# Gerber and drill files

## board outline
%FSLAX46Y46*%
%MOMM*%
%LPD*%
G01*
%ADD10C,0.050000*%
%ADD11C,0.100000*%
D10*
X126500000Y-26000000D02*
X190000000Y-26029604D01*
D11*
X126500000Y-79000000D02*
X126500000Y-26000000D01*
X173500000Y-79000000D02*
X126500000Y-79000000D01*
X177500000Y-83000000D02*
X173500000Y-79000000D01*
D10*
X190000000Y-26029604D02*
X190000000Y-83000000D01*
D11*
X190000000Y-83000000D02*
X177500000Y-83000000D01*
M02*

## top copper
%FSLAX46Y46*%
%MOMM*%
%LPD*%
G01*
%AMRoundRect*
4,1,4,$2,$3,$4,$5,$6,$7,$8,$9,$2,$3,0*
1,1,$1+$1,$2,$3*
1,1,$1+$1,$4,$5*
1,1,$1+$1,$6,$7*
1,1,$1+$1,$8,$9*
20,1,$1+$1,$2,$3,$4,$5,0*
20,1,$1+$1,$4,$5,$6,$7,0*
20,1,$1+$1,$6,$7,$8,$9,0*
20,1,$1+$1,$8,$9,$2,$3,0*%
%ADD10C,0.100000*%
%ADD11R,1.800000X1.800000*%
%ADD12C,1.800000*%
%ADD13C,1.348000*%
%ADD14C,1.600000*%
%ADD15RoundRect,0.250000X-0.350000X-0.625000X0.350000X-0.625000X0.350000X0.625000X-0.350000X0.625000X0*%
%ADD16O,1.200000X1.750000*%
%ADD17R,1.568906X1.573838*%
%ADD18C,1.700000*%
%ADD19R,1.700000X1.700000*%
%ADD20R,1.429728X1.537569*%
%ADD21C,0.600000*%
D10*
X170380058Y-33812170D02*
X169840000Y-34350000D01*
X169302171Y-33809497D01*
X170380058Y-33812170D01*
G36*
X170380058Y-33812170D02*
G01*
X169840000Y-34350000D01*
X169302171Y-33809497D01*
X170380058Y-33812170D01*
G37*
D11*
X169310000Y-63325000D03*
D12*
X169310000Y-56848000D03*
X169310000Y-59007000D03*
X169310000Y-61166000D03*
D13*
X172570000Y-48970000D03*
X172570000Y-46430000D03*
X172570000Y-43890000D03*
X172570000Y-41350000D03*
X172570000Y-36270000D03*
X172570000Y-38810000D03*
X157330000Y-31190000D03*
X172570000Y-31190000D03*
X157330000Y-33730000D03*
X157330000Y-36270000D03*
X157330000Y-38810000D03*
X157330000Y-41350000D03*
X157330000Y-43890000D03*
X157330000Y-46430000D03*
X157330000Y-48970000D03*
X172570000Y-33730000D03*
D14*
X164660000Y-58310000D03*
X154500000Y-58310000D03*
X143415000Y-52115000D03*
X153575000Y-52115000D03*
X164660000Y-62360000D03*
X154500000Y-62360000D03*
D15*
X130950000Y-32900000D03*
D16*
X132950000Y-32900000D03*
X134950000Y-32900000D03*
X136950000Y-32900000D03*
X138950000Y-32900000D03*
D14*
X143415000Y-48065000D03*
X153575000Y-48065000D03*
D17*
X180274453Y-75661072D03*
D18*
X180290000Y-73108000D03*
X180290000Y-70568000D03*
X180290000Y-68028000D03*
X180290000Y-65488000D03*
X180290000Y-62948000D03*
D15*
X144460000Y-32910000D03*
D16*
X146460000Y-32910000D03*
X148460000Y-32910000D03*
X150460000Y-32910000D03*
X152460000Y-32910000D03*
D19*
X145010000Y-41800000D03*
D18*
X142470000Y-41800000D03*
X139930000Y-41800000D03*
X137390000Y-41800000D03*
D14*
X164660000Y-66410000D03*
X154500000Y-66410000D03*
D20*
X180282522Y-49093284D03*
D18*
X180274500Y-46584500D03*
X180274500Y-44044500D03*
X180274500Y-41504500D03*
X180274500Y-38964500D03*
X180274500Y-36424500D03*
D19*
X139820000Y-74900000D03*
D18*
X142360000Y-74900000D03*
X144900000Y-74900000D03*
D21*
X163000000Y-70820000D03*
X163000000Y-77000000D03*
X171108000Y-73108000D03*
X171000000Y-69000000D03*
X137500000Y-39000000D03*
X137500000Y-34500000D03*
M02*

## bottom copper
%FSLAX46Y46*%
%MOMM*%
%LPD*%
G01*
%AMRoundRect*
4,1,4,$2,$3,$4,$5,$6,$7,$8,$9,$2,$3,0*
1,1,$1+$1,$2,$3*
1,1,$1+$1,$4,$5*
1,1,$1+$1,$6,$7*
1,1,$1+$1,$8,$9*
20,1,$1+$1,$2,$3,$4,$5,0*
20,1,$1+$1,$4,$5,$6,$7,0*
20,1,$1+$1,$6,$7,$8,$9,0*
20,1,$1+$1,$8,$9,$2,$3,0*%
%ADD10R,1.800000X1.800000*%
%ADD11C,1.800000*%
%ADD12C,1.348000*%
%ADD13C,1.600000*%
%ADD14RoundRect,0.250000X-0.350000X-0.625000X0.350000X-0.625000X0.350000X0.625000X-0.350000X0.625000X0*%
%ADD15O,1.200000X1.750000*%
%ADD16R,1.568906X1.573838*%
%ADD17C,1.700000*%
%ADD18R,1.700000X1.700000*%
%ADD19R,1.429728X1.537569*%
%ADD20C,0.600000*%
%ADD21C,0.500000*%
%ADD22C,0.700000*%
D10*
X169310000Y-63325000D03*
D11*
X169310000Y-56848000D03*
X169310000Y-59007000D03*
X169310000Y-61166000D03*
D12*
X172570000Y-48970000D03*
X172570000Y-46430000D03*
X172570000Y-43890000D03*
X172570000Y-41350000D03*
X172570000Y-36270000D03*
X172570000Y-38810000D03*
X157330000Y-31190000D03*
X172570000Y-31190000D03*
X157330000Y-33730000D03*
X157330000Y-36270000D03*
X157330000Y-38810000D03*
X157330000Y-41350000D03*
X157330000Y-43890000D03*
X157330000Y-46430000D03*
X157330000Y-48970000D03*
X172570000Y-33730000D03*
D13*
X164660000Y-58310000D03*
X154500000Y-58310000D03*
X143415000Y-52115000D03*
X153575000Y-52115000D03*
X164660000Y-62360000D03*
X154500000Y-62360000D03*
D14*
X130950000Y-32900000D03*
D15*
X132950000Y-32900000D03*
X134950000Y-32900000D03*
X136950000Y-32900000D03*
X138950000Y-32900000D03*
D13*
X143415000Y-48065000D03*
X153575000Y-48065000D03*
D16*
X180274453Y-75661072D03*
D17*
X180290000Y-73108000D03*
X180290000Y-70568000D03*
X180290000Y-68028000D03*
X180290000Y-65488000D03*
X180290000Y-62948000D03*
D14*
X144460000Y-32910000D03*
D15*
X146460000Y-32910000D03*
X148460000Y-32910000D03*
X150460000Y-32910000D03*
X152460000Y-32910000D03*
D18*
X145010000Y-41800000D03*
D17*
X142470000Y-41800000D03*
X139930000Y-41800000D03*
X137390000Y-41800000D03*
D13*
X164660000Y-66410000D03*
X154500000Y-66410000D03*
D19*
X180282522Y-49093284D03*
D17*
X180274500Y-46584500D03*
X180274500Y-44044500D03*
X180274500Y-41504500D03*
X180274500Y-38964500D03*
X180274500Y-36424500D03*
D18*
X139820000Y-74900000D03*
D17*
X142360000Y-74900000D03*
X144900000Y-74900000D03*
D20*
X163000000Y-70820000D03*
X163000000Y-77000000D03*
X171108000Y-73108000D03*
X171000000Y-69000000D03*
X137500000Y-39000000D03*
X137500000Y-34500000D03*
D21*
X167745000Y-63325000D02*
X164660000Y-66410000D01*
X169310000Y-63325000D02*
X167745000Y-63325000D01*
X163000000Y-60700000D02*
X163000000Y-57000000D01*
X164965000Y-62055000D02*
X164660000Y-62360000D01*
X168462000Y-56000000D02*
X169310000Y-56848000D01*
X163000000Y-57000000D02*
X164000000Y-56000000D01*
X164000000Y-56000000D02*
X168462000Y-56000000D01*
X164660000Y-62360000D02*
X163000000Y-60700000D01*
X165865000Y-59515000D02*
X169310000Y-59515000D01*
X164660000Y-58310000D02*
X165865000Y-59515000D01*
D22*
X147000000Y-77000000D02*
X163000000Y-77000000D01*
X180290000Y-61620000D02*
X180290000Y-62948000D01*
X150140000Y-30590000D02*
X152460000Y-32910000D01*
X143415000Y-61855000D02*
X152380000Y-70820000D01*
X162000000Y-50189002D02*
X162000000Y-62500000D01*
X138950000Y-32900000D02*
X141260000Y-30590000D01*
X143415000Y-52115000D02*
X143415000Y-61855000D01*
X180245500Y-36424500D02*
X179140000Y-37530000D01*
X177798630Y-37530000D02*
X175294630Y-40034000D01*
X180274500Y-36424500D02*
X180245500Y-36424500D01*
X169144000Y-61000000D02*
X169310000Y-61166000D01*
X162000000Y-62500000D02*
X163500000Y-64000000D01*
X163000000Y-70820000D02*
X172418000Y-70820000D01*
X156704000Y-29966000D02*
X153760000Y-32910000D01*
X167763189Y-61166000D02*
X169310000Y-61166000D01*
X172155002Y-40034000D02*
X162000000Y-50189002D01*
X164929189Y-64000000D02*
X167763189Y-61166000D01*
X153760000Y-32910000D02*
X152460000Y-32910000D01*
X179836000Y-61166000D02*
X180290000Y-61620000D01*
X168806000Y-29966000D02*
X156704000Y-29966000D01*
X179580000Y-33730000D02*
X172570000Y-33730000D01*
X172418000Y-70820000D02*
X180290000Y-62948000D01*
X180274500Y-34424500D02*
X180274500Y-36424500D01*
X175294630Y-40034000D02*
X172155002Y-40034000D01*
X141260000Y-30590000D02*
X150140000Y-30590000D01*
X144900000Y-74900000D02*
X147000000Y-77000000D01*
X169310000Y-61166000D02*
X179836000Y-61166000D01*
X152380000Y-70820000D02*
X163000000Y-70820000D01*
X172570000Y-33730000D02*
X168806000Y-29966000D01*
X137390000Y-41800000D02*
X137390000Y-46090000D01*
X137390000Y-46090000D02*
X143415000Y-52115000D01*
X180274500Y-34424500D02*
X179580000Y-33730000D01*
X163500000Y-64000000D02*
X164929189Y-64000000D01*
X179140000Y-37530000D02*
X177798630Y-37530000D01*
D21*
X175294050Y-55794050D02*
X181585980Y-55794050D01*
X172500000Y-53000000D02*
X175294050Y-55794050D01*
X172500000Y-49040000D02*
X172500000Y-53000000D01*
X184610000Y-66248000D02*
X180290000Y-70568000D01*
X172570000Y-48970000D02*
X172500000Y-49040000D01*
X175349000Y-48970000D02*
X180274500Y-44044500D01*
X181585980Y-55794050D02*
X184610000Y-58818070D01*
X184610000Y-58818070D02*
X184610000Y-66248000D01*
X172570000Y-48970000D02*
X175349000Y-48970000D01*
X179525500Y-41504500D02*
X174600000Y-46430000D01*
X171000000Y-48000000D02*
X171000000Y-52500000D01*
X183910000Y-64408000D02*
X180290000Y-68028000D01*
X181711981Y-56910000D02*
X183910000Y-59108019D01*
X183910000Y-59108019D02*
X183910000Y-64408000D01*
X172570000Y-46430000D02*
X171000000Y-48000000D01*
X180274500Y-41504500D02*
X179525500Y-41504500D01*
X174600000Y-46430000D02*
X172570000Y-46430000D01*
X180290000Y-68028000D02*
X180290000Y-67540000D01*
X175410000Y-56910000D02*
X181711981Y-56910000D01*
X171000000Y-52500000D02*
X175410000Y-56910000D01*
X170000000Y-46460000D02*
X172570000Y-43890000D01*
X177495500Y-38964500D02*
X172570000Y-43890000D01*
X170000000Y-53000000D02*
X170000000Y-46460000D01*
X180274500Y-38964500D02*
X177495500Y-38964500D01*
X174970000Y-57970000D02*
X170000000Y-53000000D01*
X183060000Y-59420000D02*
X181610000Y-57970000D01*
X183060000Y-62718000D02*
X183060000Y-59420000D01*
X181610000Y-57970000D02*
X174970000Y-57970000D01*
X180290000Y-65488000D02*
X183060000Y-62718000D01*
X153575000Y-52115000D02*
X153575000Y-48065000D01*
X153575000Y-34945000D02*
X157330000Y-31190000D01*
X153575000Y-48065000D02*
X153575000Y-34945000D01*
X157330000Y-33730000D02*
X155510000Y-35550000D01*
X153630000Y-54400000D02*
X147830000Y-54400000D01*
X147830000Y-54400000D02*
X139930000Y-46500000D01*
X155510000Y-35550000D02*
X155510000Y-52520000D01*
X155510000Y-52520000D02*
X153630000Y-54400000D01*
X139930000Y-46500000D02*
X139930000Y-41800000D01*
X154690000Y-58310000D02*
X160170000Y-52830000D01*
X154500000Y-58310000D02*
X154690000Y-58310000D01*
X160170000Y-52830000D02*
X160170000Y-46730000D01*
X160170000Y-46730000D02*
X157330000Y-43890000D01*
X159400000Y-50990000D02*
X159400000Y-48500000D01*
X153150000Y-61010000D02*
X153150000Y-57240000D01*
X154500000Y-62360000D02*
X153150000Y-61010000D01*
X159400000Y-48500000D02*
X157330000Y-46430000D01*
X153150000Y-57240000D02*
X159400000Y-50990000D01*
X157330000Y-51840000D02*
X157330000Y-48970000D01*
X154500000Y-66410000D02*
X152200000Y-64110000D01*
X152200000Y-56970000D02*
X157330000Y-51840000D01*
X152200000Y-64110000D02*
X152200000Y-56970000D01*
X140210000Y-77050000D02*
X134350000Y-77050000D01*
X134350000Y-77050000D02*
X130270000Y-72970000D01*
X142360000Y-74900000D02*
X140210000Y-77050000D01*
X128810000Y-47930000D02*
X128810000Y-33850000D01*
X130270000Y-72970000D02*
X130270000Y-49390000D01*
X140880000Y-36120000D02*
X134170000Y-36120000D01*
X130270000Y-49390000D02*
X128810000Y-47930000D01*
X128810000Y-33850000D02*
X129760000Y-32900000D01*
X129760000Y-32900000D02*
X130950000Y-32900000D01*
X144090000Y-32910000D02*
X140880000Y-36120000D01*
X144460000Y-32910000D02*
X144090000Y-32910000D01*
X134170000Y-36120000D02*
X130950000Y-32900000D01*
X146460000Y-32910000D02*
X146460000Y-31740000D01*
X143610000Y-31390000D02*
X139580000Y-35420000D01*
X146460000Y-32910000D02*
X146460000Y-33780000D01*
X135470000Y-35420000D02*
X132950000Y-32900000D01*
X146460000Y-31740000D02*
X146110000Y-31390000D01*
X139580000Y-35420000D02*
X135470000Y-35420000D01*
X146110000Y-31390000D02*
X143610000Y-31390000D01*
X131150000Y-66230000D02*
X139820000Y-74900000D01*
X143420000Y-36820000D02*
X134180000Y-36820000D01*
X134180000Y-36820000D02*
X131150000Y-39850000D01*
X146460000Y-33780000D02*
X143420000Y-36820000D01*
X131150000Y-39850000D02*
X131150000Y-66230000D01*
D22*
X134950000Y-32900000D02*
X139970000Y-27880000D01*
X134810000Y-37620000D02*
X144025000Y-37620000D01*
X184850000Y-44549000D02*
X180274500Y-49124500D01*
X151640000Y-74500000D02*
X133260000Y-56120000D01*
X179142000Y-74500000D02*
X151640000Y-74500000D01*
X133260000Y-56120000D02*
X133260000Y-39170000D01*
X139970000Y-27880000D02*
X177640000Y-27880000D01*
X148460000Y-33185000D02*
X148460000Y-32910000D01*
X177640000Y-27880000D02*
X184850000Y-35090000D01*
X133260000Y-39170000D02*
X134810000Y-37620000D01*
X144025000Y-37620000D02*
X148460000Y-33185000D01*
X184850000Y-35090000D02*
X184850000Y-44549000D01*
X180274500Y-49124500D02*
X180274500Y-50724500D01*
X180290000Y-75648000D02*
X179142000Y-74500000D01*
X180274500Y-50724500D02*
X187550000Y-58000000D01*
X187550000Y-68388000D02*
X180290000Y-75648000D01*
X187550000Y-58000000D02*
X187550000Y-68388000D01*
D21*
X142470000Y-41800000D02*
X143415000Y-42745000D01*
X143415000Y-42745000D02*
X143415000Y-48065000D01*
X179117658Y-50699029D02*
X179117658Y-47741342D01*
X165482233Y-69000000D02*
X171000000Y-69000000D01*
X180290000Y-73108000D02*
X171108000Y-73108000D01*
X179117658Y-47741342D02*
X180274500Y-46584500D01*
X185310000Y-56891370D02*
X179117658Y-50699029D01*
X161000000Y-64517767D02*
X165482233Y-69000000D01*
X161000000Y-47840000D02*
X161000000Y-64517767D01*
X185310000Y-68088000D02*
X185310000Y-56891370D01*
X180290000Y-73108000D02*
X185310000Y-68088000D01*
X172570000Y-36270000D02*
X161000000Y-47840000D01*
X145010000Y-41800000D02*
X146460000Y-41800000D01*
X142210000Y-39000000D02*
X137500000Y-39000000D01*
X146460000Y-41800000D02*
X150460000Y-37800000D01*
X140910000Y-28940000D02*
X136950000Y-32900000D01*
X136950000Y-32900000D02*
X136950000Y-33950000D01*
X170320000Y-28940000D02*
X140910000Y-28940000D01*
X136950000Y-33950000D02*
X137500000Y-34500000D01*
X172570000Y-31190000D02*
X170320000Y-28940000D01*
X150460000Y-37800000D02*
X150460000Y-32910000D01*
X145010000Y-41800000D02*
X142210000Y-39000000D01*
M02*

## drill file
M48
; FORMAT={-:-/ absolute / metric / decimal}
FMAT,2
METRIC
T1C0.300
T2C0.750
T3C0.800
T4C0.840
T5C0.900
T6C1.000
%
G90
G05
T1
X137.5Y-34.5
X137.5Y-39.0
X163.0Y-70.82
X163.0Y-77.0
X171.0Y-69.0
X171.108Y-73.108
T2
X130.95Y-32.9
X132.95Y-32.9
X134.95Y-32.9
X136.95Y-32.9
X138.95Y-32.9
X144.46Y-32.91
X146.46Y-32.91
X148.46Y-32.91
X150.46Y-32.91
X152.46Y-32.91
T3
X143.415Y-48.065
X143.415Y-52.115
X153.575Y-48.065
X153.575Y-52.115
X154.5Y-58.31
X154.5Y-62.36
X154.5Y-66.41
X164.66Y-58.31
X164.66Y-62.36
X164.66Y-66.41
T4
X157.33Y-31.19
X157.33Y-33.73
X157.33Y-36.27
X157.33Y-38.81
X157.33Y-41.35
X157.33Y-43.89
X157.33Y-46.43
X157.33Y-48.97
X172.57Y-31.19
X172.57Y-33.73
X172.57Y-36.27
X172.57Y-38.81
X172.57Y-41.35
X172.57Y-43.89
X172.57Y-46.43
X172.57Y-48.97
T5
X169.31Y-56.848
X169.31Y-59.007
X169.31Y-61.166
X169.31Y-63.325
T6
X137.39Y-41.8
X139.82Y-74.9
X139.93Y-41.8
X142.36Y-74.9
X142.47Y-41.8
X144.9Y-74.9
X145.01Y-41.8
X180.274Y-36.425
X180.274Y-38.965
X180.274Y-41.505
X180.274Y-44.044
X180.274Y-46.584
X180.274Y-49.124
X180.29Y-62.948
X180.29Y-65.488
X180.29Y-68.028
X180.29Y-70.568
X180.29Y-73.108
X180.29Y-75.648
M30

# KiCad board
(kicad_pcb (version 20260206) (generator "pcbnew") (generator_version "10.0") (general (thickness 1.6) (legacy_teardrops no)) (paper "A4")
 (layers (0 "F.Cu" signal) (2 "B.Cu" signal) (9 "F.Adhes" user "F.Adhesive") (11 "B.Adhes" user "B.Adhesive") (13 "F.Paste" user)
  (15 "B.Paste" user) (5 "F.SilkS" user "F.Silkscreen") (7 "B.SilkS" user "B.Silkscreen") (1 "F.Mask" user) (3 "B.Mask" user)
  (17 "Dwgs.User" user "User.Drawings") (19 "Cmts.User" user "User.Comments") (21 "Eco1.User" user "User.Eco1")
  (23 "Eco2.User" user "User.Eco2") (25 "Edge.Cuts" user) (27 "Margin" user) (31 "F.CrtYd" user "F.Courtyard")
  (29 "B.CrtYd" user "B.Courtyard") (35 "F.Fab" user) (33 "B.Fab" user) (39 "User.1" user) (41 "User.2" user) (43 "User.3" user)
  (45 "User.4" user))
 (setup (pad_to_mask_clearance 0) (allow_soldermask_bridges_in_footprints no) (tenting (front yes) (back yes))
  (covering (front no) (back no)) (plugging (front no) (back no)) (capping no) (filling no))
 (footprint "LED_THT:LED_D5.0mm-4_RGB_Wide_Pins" (layer "F.Cu") (at 169.31 63.325 90)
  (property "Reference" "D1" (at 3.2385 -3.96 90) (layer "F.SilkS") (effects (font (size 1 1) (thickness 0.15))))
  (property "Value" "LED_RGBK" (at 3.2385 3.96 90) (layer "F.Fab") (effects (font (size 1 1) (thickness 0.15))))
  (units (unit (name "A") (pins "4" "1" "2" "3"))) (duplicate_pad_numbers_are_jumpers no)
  (pad "1" thru_hole rect (at 0 0 90) (size 1.8 1.8) (drill 0.9) (layers "*.Cu" "*.Mask") (remove_unused_layers no) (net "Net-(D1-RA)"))
  (pad "2" thru_hole circle (at 6.477 0 90) (size 1.8 1.8) (drill 0.9) (layers "*.Cu" "*.Mask") (remove_unused_layers no)
   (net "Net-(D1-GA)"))
  (pad "3" thru_hole circle (at 4.318 0 90) (size 1.8 1.8) (drill 0.9) (layers "*.Cu" "*.Mask") (remove_unused_layers no)
   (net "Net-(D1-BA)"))
  (pad "4" thru_hole circle (at 2.159 0 90) (size 1.8 1.8) (drill 0.9) (layers "*.Cu" "*.Mask") (remove_unused_layers no) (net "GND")))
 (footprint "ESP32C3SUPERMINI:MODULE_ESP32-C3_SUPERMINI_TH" (layer "F.Cu") (at 164.95 41.09)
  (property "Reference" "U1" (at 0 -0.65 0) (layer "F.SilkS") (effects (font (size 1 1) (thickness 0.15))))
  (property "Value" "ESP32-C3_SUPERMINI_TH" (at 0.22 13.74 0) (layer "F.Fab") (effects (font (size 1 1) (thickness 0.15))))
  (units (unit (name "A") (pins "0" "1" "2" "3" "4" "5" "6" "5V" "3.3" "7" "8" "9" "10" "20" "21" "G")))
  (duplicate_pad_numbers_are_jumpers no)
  (pad "0" thru_hole circle (at 7.62 7.88) (size 1.348 1.348) (drill 0.84) (layers "*.Cu" "*.Mask") (remove_unused_layers no) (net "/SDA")
   (solder_mask_margin 0.102))
  (pad "1" thru_hole circle (at 7.62 5.34) (size 1.348 1.348) (drill 0.84) (layers "*.Cu" "*.Mask") (remove_unused_layers no) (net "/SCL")
   (solder_mask_margin 0.102))
  (pad "2" thru_hole circle (at 7.62 2.8) (size 1.348 1.348) (drill 0.84) (layers "*.Cu" "*.Mask") (remove_unused_layers no) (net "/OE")
   (solder_mask_margin 0.102))
  (pad "3" thru_hole circle (at 7.62 0.26) (size 1.348 1.348) (drill 0.84) (layers "*.Cu" "*.Mask") (remove_unused_layers no)
   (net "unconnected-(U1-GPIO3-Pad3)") (solder_mask_margin 0.102))
  (pad "3.3" thru_hole circle (at 7.62 -4.82) (size 1.348 1.348) (drill 0.84) (layers "*.Cu" "*.Mask") (remove_unused_layers no)
   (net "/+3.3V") (solder_mask_margin 0.102))
  (pad "4" thru_hole circle (at 7.62 -2.28) (size 1.348 1.348) (drill 0.84) (layers "*.Cu" "*.Mask") (remove_unused_layers no)
   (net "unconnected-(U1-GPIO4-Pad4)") (solder_mask_margin 0.102))
  (pad "5" thru_hole circle (at -7.62 -9.9) (size 1.348 1.348) (drill 0.84) (layers "*.Cu" "*.Mask") (remove_unused_layers no)
   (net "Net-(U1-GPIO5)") (solder_mask_margin 0.102))
  (pad "5V" thru_hole circle (at 7.62 -9.9) (size 1.348 1.348) (drill 0.84) (layers "*.Cu" "*.Mask") (remove_unused_layers no) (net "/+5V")
   (solder_mask_margin 0.102))
  (pad "6" thru_hole circle (at -7.62 -7.36) (size 1.348 1.348) (drill 0.84) (layers "*.Cu" "*.Mask") (remove_unused_layers no)
   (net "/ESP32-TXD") (solder_mask_margin 0.102))
  (pad "7" thru_hole circle (at -7.62 -4.82) (size 1.348 1.348) (drill 0.84) (layers "*.Cu" "*.Mask") (remove_unused_layers no)
   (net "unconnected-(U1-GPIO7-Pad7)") (solder_mask_margin 0.102))
  (pad "8" thru_hole circle (at -7.62 -2.28) (size 1.348 1.348) (drill 0.84) (layers "*.Cu" "*.Mask") (remove_unused_layers no)
   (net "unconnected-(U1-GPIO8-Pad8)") (solder_mask_margin 0.102))
  (pad "9" thru_hole circle (at -7.62 0.26) (size 1.348 1.348) (drill 0.84) (layers "*.Cu" "*.Mask") (remove_unused_layers no)
   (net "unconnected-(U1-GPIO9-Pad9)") (solder_mask_margin 0.102))
  (pad "10" thru_hole circle (at -7.62 2.8) (size 1.348 1.348) (drill 0.84) (layers "*.Cu" "*.Mask") (remove_unused_layers no) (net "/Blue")
   (solder_mask_margin 0.102))
  (pad "20" thru_hole circle (at -7.62 5.34) (size 1.348 1.348) (drill 0.84) (layers "*.Cu" "*.Mask") (remove_unused_layers no)
   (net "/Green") (solder_mask_margin 0.102))
  (pad "21" thru_hole circle (at -7.62 7.88) (size 1.348 1.348) (drill 0.84) (layers "*.Cu" "*.Mask") (remove_unused_layers no) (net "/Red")
   (solder_mask_margin 0.102))
  (pad "G" thru_hole circle (at 7.62 -7.36) (size 1.348 1.348) (drill 0.84) (layers "*.Cu" "*.Mask") (remove_unused_layers no) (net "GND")
   (solder_mask_margin 0.102)))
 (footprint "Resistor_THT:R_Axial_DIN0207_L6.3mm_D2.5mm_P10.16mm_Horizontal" (layer "F.Cu") (at 164.66 58.31 180)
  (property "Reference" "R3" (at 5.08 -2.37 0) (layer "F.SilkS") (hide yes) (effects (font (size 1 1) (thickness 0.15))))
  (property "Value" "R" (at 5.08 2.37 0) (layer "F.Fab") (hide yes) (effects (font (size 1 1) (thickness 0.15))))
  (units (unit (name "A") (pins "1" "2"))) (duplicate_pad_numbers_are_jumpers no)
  (pad "1" thru_hole circle (at 0 0 180) (size 1.6 1.6) (drill 0.8) (layers "*.Cu" "*.Mask") (remove_unused_layers no) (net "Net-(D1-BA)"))
  (pad "2" thru_hole circle (at 10.16 0 180) (size 1.6 1.6) (drill 0.8) (layers "*.Cu" "*.Mask") (remove_unused_layers no) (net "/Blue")))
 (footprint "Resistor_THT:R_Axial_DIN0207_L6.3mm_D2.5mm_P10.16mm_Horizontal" (layer "F.Cu") (at 143.415 52.115)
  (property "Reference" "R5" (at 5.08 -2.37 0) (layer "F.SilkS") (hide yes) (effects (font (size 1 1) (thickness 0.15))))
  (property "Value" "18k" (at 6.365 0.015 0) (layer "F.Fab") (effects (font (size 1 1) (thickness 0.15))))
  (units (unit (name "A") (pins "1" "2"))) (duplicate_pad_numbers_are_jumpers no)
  (pad "1" thru_hole circle (at 0 0) (size 1.6 1.6) (drill 0.8) (layers "*.Cu" "*.Mask") (remove_unused_layers no) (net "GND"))
  (pad "2" thru_hole circle (at 10.16 0) (size 1.6 1.6) (drill 0.8) (layers "*.Cu" "*.Mask") (remove_unused_layers no)
   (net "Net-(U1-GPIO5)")))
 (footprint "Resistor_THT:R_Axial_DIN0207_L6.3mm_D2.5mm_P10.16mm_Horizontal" (layer "F.Cu") (at 164.66 62.36 180)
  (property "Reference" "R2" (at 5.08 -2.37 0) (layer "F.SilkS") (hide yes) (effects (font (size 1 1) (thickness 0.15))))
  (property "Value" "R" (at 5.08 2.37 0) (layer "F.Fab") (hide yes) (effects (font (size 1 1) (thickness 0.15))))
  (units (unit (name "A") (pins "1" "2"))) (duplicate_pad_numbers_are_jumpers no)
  (pad "1" thru_hole circle (at 0 0 180) (size 1.6 1.6) (drill 0.8) (layers "*.Cu" "*.Mask") (remove_unused_layers no) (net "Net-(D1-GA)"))
  (pad "2" thru_hole circle (at 10.16 0 180) (size 1.6 1.6) (drill 0.8) (layers "*.Cu" "*.Mask") (remove_unused_layers no) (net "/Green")))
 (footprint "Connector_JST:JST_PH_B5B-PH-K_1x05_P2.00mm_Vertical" (layer "F.Cu") (at 130.95 32.9)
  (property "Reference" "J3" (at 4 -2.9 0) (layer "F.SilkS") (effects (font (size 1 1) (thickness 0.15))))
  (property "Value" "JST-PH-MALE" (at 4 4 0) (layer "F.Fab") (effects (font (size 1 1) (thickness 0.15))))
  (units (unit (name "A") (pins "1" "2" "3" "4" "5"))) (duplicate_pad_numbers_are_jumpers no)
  (pad "1" thru_hole roundrect (at 0 0) (size 1.2 1.75) (drill 0.75) (layers "*.Cu" "*.Mask") (remove_unused_layers no)
   (roundrect_rratio 0.208333) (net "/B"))
  (pad "2" thru_hole oval (at 2 0) (size 1.2 1.75) (drill 0.75) (layers "*.Cu" "*.Mask") (remove_unused_layers no) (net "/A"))
  (pad "3" thru_hole oval (at 4 0) (size 1.2 1.75) (drill 0.75) (layers "*.Cu" "*.Mask") (remove_unused_layers no) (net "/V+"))
  (pad "4" thru_hole oval (at 6 0) (size 1.2 1.75) (drill 0.75) (layers "*.Cu" "*.Mask") (remove_unused_layers no) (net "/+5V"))
  (pad "5" thru_hole oval (at 8 0) (size 1.2 1.75) (drill 0.75) (layers "*.Cu" "*.Mask") (remove_unused_layers no) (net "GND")))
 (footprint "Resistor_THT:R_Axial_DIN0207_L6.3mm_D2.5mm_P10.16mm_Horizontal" (layer "F.Cu") (at 143.415 48.065)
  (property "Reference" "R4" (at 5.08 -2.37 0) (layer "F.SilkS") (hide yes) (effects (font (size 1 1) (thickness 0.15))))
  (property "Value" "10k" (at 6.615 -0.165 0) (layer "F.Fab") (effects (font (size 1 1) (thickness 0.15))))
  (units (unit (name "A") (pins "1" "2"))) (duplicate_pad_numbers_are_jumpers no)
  (pad "1" thru_hole circle (at 0 0) (size 1.6 1.6) (drill 0.8) (layers "*.Cu" "*.Mask") (remove_unused_layers no) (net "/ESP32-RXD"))
  (pad "2" thru_hole circle (at 10.16 0) (size 1.6 1.6) (drill 0.8) (layers "*.Cu" "*.Mask") (remove_unused_layers no)
   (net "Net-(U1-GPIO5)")))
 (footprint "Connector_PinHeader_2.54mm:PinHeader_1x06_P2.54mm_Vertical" (layer "F.Cu") (at 180.29 75.648 180)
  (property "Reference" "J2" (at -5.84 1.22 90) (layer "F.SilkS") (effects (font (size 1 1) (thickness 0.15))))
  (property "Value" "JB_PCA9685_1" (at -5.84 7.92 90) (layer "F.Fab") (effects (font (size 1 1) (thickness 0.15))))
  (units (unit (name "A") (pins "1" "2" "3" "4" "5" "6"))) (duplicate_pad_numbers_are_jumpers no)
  (pad "1" thru_hole rect (at 0 0 180) (size 1.568906 1.573838) (drill 1 (offset 0.015547 -0.013072)) (layers "*.Cu" "*.Mask")
   (remove_unused_layers no) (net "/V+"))
  (pad "2" thru_hole circle (at 0 2.54 180) (size 1.7 1.7) (drill 1) (layers "*.Cu" "*.Mask") (remove_unused_layers no) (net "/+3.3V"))
  (pad "3" thru_hole circle (at 0 5.08 180) (size 1.7 1.7) (drill 1) (layers "*.Cu" "*.Mask") (remove_unused_layers no) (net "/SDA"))
  (pad "4" thru_hole circle (at 0 7.62 180) (size 1.7 1.7) (drill 1) (layers "*.Cu" "*.Mask") (remove_unused_layers no) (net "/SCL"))
  (pad "5" thru_hole circle (at 0 10.16 180) (size 1.7 1.7) (drill 1) (layers "*.Cu" "*.Mask") (remove_unused_layers no) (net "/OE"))
  (pad "6" thru_hole circle (at 0 12.7 180) (size 1.7 1.7) (drill 1) (layers "*.Cu" "*.Mask") (remove_unused_layers no) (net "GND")))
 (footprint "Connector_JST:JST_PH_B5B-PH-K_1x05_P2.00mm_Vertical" (layer "F.Cu") (at 144.46 32.91)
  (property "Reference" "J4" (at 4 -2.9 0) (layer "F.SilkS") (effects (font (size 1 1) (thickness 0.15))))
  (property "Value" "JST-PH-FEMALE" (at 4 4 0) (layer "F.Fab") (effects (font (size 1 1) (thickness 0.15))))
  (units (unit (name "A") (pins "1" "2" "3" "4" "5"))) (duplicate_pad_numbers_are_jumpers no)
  (pad "1" thru_hole roundrect (at 0 0) (size 1.2 1.75) (drill 0.75) (layers "*.Cu" "*.Mask") (remove_unused_layers no)
   (roundrect_rratio 0.208333) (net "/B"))
  (pad "2" thru_hole oval (at 2 0) (size 1.2 1.75) (drill 0.75) (layers "*.Cu" "*.Mask") (remove_unused_layers no) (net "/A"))
  (pad "3" thru_hole oval (at 4 0) (size 1.2 1.75) (drill 0.75) (layers "*.Cu" "*.Mask") (remove_unused_layers no) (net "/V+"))
  (pad "4" thru_hole oval (at 6 0) (size 1.2 1.75) (drill 0.75) (layers "*.Cu" "*.Mask") (remove_unused_layers no) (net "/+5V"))
  (pad "5" thru_hole oval (at 8 0) (size 1.2 1.75) (drill 0.75) (layers "*.Cu" "*.Mask") (remove_unused_layers no) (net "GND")))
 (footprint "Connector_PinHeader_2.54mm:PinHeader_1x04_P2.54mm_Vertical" (layer "F.Cu") (at 145.01 41.8 -90)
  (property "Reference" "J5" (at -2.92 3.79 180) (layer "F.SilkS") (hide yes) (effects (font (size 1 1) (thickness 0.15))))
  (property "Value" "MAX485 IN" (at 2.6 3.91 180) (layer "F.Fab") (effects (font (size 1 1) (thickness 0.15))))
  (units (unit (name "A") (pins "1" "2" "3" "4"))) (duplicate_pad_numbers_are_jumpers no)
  (pad "1" thru_hole rect (at 0 0 270) (size 1.7 1.7) (drill 1) (layers "*.Cu" "*.Mask") (remove_unused_layers no) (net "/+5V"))
  (pad "2" thru_hole circle (at 0 2.54 270) (size 1.7 1.7) (drill 1) (layers "*.Cu" "*.Mask") (remove_unused_layers no) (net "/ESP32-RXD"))
  (pad "3" thru_hole circle (at 0 5.08 270) (size 1.7 1.7) (drill 1) (layers "*.Cu" "*.Mask") (remove_unused_layers no) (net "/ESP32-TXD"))
  (pad "4" thru_hole circle (at 0 7.62 270) (size 1.7 1.7) (drill 1) (layers "*.Cu" "*.Mask") (remove_unused_layers no) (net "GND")))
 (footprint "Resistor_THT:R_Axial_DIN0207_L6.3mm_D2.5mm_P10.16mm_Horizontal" (layer "F.Cu") (at 164.66 66.41 180)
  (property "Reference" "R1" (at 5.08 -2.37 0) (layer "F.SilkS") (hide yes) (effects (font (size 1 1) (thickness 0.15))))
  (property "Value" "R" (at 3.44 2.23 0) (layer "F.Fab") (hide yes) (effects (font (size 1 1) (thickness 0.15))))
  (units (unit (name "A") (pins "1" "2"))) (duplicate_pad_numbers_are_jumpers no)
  (pad "1" thru_hole circle (at 0 0 180) (size 1.6 1.6) (drill 0.8) (layers "*.Cu" "*.Mask") (remove_unused_layers no) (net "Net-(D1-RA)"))
  (pad "2" thru_hole circle (at 10.16 0 180) (size 1.6 1.6) (drill 0.8) (layers "*.Cu" "*.Mask") (remove_unused_layers no) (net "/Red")))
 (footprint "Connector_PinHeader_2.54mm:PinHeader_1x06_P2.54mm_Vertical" (layer "F.Cu") (at 180.2745 49.1245 180)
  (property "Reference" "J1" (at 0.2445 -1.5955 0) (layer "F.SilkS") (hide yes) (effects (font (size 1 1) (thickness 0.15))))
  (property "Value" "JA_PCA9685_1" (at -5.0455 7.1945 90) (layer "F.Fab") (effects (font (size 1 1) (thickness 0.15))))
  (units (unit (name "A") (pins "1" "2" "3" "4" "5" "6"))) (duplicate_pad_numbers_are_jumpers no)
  (pad "1" thru_hole rect (at 0 0 180) (size 1.429728 1.537569) (drill 1 (offset -0.008022 0.031216)) (layers "*.Cu" "*.Mask")
   (remove_unused_layers no) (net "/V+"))
  (pad "2" thru_hole circle (at 0 2.54 180) (size 1.7 1.7) (drill 1) (layers "*.Cu" "*.Mask") (remove_unused_layers no) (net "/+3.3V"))
  (pad "3" thru_hole circle (at 0 5.08 180) (size 1.7 1.7) (drill 1) (layers "*.Cu" "*.Mask") (remove_unused_layers no) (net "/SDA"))
  (pad "4" thru_hole circle (at 0 7.62 180) (size 1.7 1.7) (drill 1) (layers "*.Cu" "*.Mask") (remove_unused_layers no) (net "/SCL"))
  (pad "5" thru_hole circle (at 0 10.16 180) (size 1.7 1.7) (drill 1) (layers "*.Cu" "*.Mask") (remove_unused_layers no) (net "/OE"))
  (pad "6" thru_hole circle (at 0 12.7 180) (size 1.7 1.7) (drill 1) (layers "*.Cu" "*.Mask") (remove_unused_layers no) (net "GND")))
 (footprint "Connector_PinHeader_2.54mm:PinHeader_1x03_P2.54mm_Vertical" (layer "F.Cu") (at 139.82 74.9 90)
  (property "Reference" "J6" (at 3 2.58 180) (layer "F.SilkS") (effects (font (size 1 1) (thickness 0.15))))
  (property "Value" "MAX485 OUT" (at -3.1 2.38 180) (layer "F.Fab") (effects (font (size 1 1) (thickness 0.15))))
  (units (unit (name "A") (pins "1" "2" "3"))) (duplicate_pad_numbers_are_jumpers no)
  (pad "1" thru_hole rect (at 0 0 90) (size 1.7 1.7) (drill 1) (layers "*.Cu" "*.Mask") (remove_unused_layers no) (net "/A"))
  (pad "2" thru_hole circle (at 0 2.54 90) (size 1.7 1.7) (drill 1) (layers "*.Cu" "*.Mask") (remove_unused_layers no) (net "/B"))
  (pad "3" thru_hole circle (at 0 5.08 90) (size 1.7 1.7) (drill 1) (layers "*.Cu" "*.Mask") (remove_unused_layers no) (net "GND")))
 (gr_poly
  (pts (xy 170.380058 33.81217) (xy 169.84 34.35) (xy 169.302171 33.809497)) (stroke (width 0.1) (type solid)) (fill yes) (layer "F.Cu"))
 (gr_line (start 126.5 26) (end 190 26.029604) (stroke (width 0.05) (type default)) (layer "Edge.Cuts"))
 (gr_line (start 126.5 79) (end 126.5 26) (stroke (width 0.1) (type solid)) (layer "Edge.Cuts"))
 (gr_line (start 173.5 79) (end 126.5 79) (stroke (width 0.1) (type solid)) (layer "Edge.Cuts"))
 (gr_line (start 177.5 83) (end 173.5 79) (stroke (width 0.1) (type solid)) (layer "Edge.Cuts"))
 (gr_line (start 190 26.029604) (end 190 83) (stroke (width 0.05) (type default)) (layer "Edge.Cuts"))
 (gr_line (start 190 83) (end 177.5 83) (stroke (width 0.1) (type solid)) (layer "Edge.Cuts"))
 (segment (start 167.745 63.325) (end 164.66 66.41) (width 0.5) (layer "B.Cu") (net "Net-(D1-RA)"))
 (segment (start 169.31 63.325) (end 167.745 63.325) (width 0.5) (layer "B.Cu") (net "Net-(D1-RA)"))
 (segment (start 163 60.7) (end 163 57) (width 0.5) (layer "B.Cu") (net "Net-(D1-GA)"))
 (segment (start 164.965 62.055) (end 164.66 62.36) (width 0.5) (layer "B.Cu") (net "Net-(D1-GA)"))
 (segment (start 168.462 56) (end 169.31 56.848) (width 0.5) (layer "B.Cu") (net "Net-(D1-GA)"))
 (segment (start 163 57) (end 164 56) (width 0.5) (layer "B.Cu") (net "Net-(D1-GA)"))
 (segment (start 164 56) (end 168.462 56) (width 0.5) (layer "B.Cu") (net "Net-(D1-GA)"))
 (segment (start 164.66 62.36) (end 163 60.7) (width 0.5) (layer "B.Cu") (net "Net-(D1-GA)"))
 (segment (start 165.865 59.515) (end 169.31 59.515) (width 0.5) (layer "B.Cu") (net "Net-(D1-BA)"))
 (segment (start 164.66 58.31) (end 165.865 59.515) (width 0.5) (layer "B.Cu") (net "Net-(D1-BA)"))
 (via (at 163 70.82) (size 0.6) (drill 0.3) (layers "F.Cu" "B.Cu") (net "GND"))
 (via (at 163 77) (size 0.6) (drill 0.3) (layers "F.Cu" "B.Cu") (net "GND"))
 (segment (start 147 77) (end 163 77) (width 0.7) (layer "B.Cu") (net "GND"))
 (segment (start 180.29 61.62) (end 180.29 62.948) (width 0.7) (layer "B.Cu") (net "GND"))
 (segment (start 150.14 30.59) (end 152.46 32.91) (width 0.7) (layer "B.Cu") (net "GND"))
 (segment (start 143.415 61.855) (end 152.38 70.82) (width 0.7) (layer "B.Cu") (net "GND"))
 (segment (start 162 50.189002) (end 162 62.5) (width 0.7) (layer "B.Cu") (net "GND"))
 (segment (start 138.95 32.9) (end 141.26 30.59) (width 0.7) (layer "B.Cu") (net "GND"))
 (segment (start 143.415 52.115) (end 143.415 61.855) (width 0.7) (layer "B.Cu") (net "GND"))
 (segment (start 180.2455 36.4245) (end 179.14 37.53) (width 0.7) (layer "B.Cu") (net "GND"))
 (segment (start 177.79863 37.53) (end 175.29463 40.034) (width 0.7) (layer "B.Cu") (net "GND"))
 (segment (start 180.2745 36.4245) (end 180.2455 36.4245) (width 0.7) (layer "B.Cu") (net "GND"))
 (segment (start 169.144 61) (end 169.31 61.166) (width 0.7) (layer "B.Cu") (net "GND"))
 (segment (start 162 62.5) (end 163.5 64) (width 0.7) (layer "B.Cu") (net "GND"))
 (segment (start 163 70.82) (end 172.418 70.82) (width 0.7) (layer "B.Cu") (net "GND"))
 (segment (start 156.704 29.966) (end 153.76 32.91) (width 0.7) (layer "B.Cu") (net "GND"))
 (segment (start 167.763189 61.166) (end 169.31 61.166) (width 0.7) (layer "B.Cu") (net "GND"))
 (segment (start 172.155002 40.034) (end 162 50.189002) (width 0.7) (layer "B.Cu") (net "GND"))
 (segment (start 164.929189 64) (end 167.763189 61.166) (width 0.7) (layer "B.Cu") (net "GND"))
 (segment (start 153.76 32.91) (end 152.46 32.91) (width 0.7) (layer "B.Cu") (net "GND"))
 (segment (start 179.836 61.166) (end 180.29 61.62) (width 0.7) (layer "B.Cu") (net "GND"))
 (segment (start 168.806 29.966) (end 156.704 29.966) (width 0.7) (layer "B.Cu") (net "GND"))
 (segment (start 179.58 33.73) (end 172.57 33.73) (width 0.7) (layer "B.Cu") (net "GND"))
 (segment (start 172.418 70.82) (end 180.29 62.948) (width 0.7) (layer "B.Cu") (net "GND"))
 (segment (start 180.2745 34.4245) (end 180.2745 36.4245) (width 0.7) (layer "B.Cu") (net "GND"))
 (segment (start 175.29463 40.034) (end 172.155002 40.034) (width 0.7) (layer "B.Cu") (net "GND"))
 (segment (start 141.26 30.59) (end 150.14 30.59) (width 0.7) (layer "B.Cu") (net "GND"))
 (segment (start 144.9 74.9) (end 147 77) (width 0.7) (layer "B.Cu") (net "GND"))
 (segment (start 169.31 61.166) (end 179.836 61.166) (width 0.7) (layer "B.Cu") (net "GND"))
 (segment (start 152.38 70.82) (end 163 70.82) (width 0.7) (layer "B.Cu") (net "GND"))
 (segment (start 172.57 33.73) (end 168.806 29.966) (width 0.7) (layer "B.Cu") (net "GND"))
 (segment (start 137.39 41.8) (end 137.39 46.09) (width 0.7) (layer "B.Cu") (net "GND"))
 (segment (start 137.39 46.09) (end 143.415 52.115) (width 0.7) (layer "B.Cu") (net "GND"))
 (segment (start 180.2745 34.4245) (end 179.58 33.73) (width 0.7) (layer "B.Cu") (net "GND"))
 (segment (start 163.5 64) (end 164.929189 64) (width 0.7) (layer "B.Cu") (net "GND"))
 (segment (start 179.14 37.53) (end 177.79863 37.53) (width 0.7) (layer "B.Cu") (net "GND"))
 (segment (start 175.29405 55.79405) (end 181.58598 55.79405) (width 0.5) (layer "B.Cu") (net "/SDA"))
 (segment (start 172.5 53) (end 175.29405 55.79405) (width 0.5) (layer "B.Cu") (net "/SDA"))
 (segment (start 172.5 49.04) (end 172.5 53) (width 0.5) (layer "B.Cu") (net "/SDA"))
 (segment (start 184.61 66.248) (end 180.29 70.568) (width 0.5) (layer "B.Cu") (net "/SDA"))
 (segment (start 172.57 48.97) (end 172.5 49.04) (width 0.5) (layer "B.Cu") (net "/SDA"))
 (segment (start 175.349 48.97) (end 180.2745 44.0445) (width 0.5) (layer "B.Cu") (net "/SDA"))
 (segment (start 181.58598 55.79405) (end 184.61 58.81807) (width 0.5) (layer "B.Cu") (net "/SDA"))
 (segment (start 184.61 58.81807) (end 184.61 66.248) (width 0.5) (layer "B.Cu") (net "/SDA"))
 (segment (start 172.57 48.97) (end 175.349 48.97) (width 0.5) (layer "B.Cu") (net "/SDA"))
 (segment (start 179.5255 41.5045) (end 174.6 46.43) (width 0.5) (layer "B.Cu") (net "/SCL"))
 (segment (start 171 48) (end 171 52.5) (width 0.5) (layer "B.Cu") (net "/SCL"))
 (segment (start 183.91 64.408) (end 180.29 68.028) (width 0.5) (layer "B.Cu") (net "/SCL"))
 (segment (start 181.711981 56.91) (end 183.91 59.108019) (width 0.5) (layer "B.Cu") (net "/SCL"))
 (segment (start 183.91 59.108019) (end 183.91 64.408) (width 0.5) (layer "B.Cu") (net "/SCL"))
 (segment (start 172.57 46.43) (end 171 48) (width 0.5) (layer "B.Cu") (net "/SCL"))
 (segment (start 180.2745 41.5045) (end 179.5255 41.5045) (width 0.5) (layer "B.Cu") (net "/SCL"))
 (segment (start 174.6 46.43) (end 172.57 46.43) (width 0.5) (layer "B.Cu") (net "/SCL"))
 (segment (start 180.29 68.028) (end 180.29 67.54) (width 0.5) (layer "B.Cu") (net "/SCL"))
 (segment (start 175.41 56.91) (end 181.711981 56.91) (width 0.5) (layer "B.Cu") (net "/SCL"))
 (segment (start 171 52.5) (end 175.41 56.91) (width 0.5) (layer "B.Cu") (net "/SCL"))
 (segment (start 170 46.46) (end 172.57 43.89) (width 0.5) (layer "B.Cu") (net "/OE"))
 (segment (start 177.4955 38.9645) (end 172.57 43.89) (width 0.5) (layer "B.Cu") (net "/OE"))
 (segment (start 170 53) (end 170 46.46) (width 0.5) (layer "B.Cu") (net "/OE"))
 (segment (start 180.2745 38.9645) (end 177.4955 38.9645) (width 0.5) (layer "B.Cu") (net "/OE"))
 (segment (start 174.97 57.97) (end 170 53) (width 0.5) (layer "B.Cu") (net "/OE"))
 (segment (start 183.06 59.42) (end 181.61 57.97) (width 0.5) (layer "B.Cu") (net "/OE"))
 (segment (start 183.06 62.718) (end 183.06 59.42) (width 0.5) (layer "B.Cu") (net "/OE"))
 (segment (start 181.61 57.97) (end 174.97 57.97) (width 0.5) (layer "B.Cu") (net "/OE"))
 (segment (start 180.29 65.488) (end 183.06 62.718) (width 0.5) (layer "B.Cu") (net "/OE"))
 (segment (start 153.575 52.115) (end 153.575 48.065) (width 0.5) (layer "B.Cu") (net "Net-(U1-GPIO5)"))
 (segment (start 153.575 34.945) (end 157.33 31.19) (width 0.5) (layer "B.Cu") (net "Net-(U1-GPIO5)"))
 (segment (start 153.575 48.065) (end 153.575 34.945) (width 0.5) (layer "B.Cu") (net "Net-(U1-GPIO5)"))
 (segment (start 157.33 33.73) (end 155.51 35.55) (width 0.5) (layer "B.Cu") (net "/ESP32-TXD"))
 (segment (start 153.63 54.4) (end 147.83 54.4) (width 0.5) (layer "B.Cu") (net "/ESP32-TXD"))
 (segment (start 147.83 54.4) (end 139.93 46.5) (width 0.5) (layer "B.Cu") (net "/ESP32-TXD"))
 (segment (start 155.51 35.55) (end 155.51 52.52) (width 0.5) (layer "B.Cu") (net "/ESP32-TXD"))
 (segment (start 155.51 52.52) (end 153.63 54.4) (width 0.5) (layer "B.Cu") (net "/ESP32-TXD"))
 (segment (start 139.93 46.5) (end 139.93 41.8) (width 0.5) (layer "B.Cu") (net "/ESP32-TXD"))
 (segment (start 154.69 58.31) (end 160.17 52.83) (width 0.5) (layer "B.Cu") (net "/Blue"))
 (segment (start 154.5 58.31) (end 154.69 58.31) (width 0.5) (layer "B.Cu") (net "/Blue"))
 (segment (start 160.17 52.83) (end 160.17 46.73) (width 0.5) (layer "B.Cu") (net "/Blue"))
 (segment (start 160.17 46.73) (end 157.33 43.89) (width 0.5) (layer "B.Cu") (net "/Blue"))
 (segment (start 159.4 50.99) (end 159.4 48.5) (width 0.5) (layer "B.Cu") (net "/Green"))
 (segment (start 153.15 61.01) (end 153.15 57.24) (width 0.5) (layer "B.Cu") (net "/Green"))
 (segment (start 154.5 62.36) (end 153.15 61.01) (width 0.5) (layer "B.Cu") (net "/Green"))
 (segment (start 159.4 48.5) (end 157.33 46.43) (width 0.5) (layer "B.Cu") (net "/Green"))
 (segment (start 153.15 57.24) (end 159.4 50.99) (width 0.5) (layer "B.Cu") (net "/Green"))
 (segment (start 157.33 51.84) (end 157.33 48.97) (width 0.5) (layer "B.Cu") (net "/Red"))
 (segment (start 154.5 66.41) (end 152.2 64.11) (width 0.5) (layer "B.Cu") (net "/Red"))
 (segment (start 152.2 56.97) (end 157.33 51.84) (width 0.5) (layer "B.Cu") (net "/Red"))
 (segment (start 152.2 64.11) (end 152.2 56.97) (width 0.5) (layer "B.Cu") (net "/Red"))
 (segment (start 140.21 77.05) (end 134.35 77.05) (width 0.5) (layer "B.Cu") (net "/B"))
 (segment (start 134.35 77.05) (end 130.27 72.97) (width 0.5) (layer "B.Cu") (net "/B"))
 (segment (start 142.36 74.9) (end 140.21 77.05) (width 0.5) (layer "B.Cu") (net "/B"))
 (segment (start 128.81 47.93) (end 128.81 33.85) (width 0.5) (layer "B.Cu") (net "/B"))
 (segment (start 130.27 72.97) (end 130.27 49.39) (width 0.5) (layer "B.Cu") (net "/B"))
 (segment (start 140.88 36.12) (end 134.17 36.12) (width 0.5) (layer "B.Cu") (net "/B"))
 (segment (start 130.27 49.39) (end 128.81 47.93) (width 0.5) (layer "B.Cu") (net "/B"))
 (segment (start 128.81 33.85) (end 129.76 32.9) (width 0.5) (layer "B.Cu") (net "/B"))
 (segment (start 129.76 32.9) (end 130.95 32.9) (width 0.5) (layer "B.Cu") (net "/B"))
 (segment (start 144.09 32.91) (end 140.88 36.12) (width 0.5) (layer "B.Cu") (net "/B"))
 (segment (start 144.46 32.91) (end 144.09 32.91) (width 0.5) (layer "B.Cu") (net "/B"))
 (segment (start 134.17 36.12) (end 130.95 32.9) (width 0.5) (layer "B.Cu") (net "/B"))
 (segment (start 146.46 32.91) (end 146.46 31.74) (width 0.5) (layer "B.Cu") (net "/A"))
 (segment (start 143.61 31.39) (end 139.58 35.42) (width 0.5) (layer "B.Cu") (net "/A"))
 (segment (start 146.46 32.91) (end 146.46 33.78) (width 0.5) (layer "B.Cu") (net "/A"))
 (segment (start 135.47 35.42) (end 132.95 32.9) (width 0.5) (layer "B.Cu") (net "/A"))
 (segment (start 146.46 31.74) (end 146.11 31.39) (width 0.5) (layer "B.Cu") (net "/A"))
 (segment (start 139.58 35.42) (end 135.47 35.42) (width 0.5) (layer "B.Cu") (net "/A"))
 (segment (start 146.11 31.39) (end 143.61 31.39) (width 0.5) (layer "B.Cu") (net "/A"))
 (segment (start 131.15 66.23) (end 139.82 74.9) (width 0.5) (layer "B.Cu") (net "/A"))
 (segment (start 143.42 36.82) (end 134.18 36.82) (width 0.5) (layer "B.Cu") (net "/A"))
 (segment (start 134.18 36.82) (end 131.15 39.85) (width 0.5) (layer "B.Cu") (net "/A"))
 (segment (start 146.46 33.78) (end 143.42 36.82) (width 0.5) (layer "B.Cu") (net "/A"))
 (segment (start 131.15 39.85) (end 131.15 66.23) (width 0.5) (layer "B.Cu") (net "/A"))
 (segment (start 134.95 32.9) (end 139.97 27.88) (width 0.7) (layer "B.Cu") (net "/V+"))
 (segment (start 134.81 37.62) (end 144.025 37.62) (width 0.7) (layer "B.Cu") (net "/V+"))
 (segment (start 184.85 44.549) (end 180.2745 49.1245) (width 0.7) (layer "B.Cu") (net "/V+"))
 (segment (start 151.64 74.5) (end 133.26 56.12) (width 0.7) (layer "B.Cu") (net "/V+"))
 (segment (start 179.142 74.5) (end 151.64 74.5) (width 0.7) (layer "B.Cu") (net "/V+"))
 (segment (start 133.26 56.12) (end 133.26 39.17) (width 0.7) (layer "B.Cu") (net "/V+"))
 (segment (start 139.97 27.88) (end 177.64 27.88) (width 0.7) (layer "B.Cu") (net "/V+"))
 (segment (start 148.46 33.185) (end 148.46 32.91) (width 0.7) (layer "B.Cu") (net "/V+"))
 (segment (start 177.64 27.88) (end 184.85 35.09) (width 0.7) (layer "B.Cu") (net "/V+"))
 (segment (start 133.26 39.17) (end 134.81 37.62) (width 0.7) (layer "B.Cu") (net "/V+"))
 (segment (start 144.025 37.62) (end 148.46 33.185) (width 0.7) (layer "B.Cu") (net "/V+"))
 (segment (start 184.85 35.09) (end 184.85 44.549) (width 0.7) (layer "B.Cu") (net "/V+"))
 (segment (start 180.2745 49.1245) (end 180.2745 50.7245) (width 0.7) (layer "B.Cu") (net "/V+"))
 (segment (start 180.29 75.648) (end 179.142 74.5) (width 0.7) (layer "B.Cu") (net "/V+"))
 (segment (start 180.2745 50.7245) (end 187.55 58) (width 0.7) (layer "B.Cu") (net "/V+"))
 (segment (start 187.55 68.388) (end 180.29 75.648) (width 0.7) (layer "B.Cu") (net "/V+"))
 (segment (start 187.55 58) (end 187.55 68.388) (width 0.7) (layer "B.Cu") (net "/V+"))
 (segment (start 142.47 41.8) (end 143.415 42.745) (width 0.5) (layer "B.Cu") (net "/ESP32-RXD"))
 (segment (start 143.415 42.745) (end 143.415 48.065) (width 0.5) (layer "B.Cu") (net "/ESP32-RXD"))
 (via (at 171.108 73.108) (size 0.6) (drill 0.3) (layers "F.Cu" "B.Cu") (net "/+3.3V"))
 (via (at 171 69) (size 0.6) (drill 0.3) (layers "F.Cu" "B.Cu") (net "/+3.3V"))
 (segment (start 179.117658 50.699029) (end 179.117658 47.741342) (width 0.5) (layer "B.Cu") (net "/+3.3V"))
 (segment (start 165.482233 69) (end 171 69) (width 0.5) (layer "B.Cu") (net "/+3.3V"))
 (segment (start 180.29 73.108) (end 171.108 73.108) (width 0.5) (layer "B.Cu") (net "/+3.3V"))
 (segment (start 179.117658 47.741342) (end 180.2745 46.5845) (width 0.5) (layer "B.Cu") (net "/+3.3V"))
 (segment (start 185.31 56.89137) (end 179.117658 50.699029) (width 0.5) (layer "B.Cu") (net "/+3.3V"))
 (segment (start 161 64.517767) (end 165.482233 69) (width 0.5) (layer "B.Cu") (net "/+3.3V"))
 (segment (start 161 47.84) (end 161 64.517767) (width 0.5) (layer "B.Cu") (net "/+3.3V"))
 (segment (start 185.31 68.088) (end 185.31 56.89137) (width 0.5) (layer "B.Cu") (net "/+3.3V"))
 (segment (start 180.29 73.108) (end 185.31 68.088) (width 0.5) (layer "B.Cu") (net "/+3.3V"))
 (segment (start 172.57 36.27) (end 161 47.84) (width 0.5) (layer "B.Cu") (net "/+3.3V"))
 (via (at 137.5 39) (size 0.6) (drill 0.3) (layers "F.Cu" "B.Cu") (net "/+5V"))
 (via (at 137.5 34.5) (size 0.6) (drill 0.3) (layers "F.Cu" "B.Cu") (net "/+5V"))
 (segment (start 145.01 41.8) (end 146.46 41.8) (width 0.5) (layer "B.Cu") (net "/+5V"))
 (segment (start 142.21 39) (end 137.5 39) (width 0.5) (layer "B.Cu") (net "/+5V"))
 (segment (start 146.46 41.8) (end 150.46 37.8) (width 0.5) (layer "B.Cu") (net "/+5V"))
 (segment (start 140.91 28.94) (end 136.95 32.9) (width 0.5) (layer "B.Cu") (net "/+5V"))
 (segment (start 136.95 32.9) (end 136.95 33.95) (width 0.5) (layer "B.Cu") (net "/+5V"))
 (segment (start 170.32 28.94) (end 140.91 28.94) (width 0.5) (layer "B.Cu") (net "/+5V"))
 (segment (start 136.95 33.95) (end 137.5 34.5) (width 0.5) (layer "B.Cu") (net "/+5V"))
 (segment (start 172.57 31.19) (end 170.32 28.94) (width 0.5) (layer "B.Cu") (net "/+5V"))
 (segment (start 150.46 37.8) (end 150.46 32.91) (width 0.5) (layer "B.Cu") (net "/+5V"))
 (segment (start 145.01 41.8) (end 142.21 39) (width 0.5) (layer "B.Cu") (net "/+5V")))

